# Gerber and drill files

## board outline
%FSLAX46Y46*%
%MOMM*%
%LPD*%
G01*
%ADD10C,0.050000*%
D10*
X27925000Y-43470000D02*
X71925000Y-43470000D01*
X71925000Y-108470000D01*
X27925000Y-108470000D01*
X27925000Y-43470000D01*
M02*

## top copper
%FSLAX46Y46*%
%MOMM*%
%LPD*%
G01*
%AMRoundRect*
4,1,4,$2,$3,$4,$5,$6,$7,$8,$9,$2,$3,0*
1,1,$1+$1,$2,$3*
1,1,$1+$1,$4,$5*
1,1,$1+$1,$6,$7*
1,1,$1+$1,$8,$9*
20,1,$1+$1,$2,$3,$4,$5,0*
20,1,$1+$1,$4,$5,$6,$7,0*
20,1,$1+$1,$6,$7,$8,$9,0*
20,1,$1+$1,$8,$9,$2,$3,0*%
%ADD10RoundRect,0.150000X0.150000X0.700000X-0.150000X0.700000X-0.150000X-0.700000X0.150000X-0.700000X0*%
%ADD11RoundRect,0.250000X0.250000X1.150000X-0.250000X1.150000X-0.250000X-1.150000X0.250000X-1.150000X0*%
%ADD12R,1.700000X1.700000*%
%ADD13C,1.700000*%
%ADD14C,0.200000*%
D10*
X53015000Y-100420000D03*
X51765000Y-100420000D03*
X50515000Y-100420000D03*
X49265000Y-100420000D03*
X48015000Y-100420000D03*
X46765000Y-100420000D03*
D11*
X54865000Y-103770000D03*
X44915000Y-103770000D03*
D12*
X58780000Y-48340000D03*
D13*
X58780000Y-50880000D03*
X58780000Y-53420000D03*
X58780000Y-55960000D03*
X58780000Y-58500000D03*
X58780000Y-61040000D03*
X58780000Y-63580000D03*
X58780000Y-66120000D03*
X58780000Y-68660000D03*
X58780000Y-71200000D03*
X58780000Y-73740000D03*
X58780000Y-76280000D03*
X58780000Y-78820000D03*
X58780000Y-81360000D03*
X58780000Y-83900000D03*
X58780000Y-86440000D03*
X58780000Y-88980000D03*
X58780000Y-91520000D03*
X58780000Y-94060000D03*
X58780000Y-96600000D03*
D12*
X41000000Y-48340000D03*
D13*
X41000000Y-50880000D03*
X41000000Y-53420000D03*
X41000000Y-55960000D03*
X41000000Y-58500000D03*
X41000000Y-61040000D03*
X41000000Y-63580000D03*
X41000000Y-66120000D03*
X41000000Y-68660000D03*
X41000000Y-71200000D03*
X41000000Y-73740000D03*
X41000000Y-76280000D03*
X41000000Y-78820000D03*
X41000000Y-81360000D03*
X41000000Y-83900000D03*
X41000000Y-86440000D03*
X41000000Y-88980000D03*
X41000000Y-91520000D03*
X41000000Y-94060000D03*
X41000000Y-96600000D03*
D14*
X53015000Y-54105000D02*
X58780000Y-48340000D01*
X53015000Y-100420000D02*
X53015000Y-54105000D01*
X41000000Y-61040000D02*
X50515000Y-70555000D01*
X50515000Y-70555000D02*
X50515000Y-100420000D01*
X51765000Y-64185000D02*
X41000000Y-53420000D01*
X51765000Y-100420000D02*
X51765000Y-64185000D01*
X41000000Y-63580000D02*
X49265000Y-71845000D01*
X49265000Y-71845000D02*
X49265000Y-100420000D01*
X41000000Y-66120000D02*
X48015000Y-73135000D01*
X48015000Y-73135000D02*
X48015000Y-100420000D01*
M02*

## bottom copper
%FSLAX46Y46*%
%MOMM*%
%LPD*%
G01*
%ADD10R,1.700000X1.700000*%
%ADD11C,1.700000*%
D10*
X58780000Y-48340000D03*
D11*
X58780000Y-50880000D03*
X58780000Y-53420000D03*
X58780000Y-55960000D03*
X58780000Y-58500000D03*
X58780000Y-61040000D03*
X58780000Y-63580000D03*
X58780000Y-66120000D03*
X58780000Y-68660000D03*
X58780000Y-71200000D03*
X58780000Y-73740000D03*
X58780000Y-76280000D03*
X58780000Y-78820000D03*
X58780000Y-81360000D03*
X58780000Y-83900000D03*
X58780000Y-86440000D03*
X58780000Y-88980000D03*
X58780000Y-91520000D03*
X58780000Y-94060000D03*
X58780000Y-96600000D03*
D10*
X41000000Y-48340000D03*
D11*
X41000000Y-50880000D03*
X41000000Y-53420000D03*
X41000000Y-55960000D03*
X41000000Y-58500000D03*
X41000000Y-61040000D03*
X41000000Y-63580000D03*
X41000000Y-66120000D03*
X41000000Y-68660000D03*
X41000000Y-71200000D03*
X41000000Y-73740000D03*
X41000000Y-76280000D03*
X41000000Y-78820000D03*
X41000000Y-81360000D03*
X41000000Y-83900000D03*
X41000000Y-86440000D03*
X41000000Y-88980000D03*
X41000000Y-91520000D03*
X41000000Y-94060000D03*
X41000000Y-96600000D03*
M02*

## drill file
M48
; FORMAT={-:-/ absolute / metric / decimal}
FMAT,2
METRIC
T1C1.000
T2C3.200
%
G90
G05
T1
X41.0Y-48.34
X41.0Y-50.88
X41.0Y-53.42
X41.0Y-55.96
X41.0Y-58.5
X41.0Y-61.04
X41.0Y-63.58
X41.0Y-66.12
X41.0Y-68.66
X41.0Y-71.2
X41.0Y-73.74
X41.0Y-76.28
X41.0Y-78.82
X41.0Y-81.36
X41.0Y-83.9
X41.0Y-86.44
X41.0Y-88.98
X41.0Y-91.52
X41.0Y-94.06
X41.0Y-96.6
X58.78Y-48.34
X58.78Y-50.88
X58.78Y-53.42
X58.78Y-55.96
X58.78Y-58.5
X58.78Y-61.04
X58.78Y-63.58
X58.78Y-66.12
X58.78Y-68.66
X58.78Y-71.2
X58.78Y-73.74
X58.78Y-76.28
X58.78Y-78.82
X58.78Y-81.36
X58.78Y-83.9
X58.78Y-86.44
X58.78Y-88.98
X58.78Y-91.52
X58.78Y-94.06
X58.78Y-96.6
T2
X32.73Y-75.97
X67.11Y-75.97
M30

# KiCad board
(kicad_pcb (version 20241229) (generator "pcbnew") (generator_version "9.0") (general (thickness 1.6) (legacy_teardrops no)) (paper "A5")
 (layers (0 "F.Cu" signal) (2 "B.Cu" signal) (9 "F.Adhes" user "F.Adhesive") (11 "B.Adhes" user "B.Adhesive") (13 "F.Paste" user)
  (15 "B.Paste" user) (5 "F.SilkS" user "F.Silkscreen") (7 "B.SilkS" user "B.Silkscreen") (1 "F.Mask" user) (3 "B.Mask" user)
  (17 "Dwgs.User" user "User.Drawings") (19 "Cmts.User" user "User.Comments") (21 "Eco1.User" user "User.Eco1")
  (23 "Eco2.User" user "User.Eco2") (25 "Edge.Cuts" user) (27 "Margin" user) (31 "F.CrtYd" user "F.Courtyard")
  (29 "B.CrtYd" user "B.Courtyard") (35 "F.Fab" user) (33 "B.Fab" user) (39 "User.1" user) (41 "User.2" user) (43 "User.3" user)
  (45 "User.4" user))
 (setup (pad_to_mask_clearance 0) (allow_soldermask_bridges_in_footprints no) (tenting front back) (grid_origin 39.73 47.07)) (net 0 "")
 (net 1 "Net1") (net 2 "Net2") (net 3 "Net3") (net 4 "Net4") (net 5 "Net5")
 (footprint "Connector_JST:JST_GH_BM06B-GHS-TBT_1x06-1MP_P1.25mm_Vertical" (layer "F.Cu") (at 49.89 102.37 180)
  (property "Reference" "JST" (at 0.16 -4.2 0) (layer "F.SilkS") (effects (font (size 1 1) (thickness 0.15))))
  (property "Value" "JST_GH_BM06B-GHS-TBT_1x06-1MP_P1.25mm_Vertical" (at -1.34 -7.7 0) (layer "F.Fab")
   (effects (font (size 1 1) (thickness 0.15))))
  (pad "1" smd roundrect (at -3.125 1.95 180) (size 0.6 1.7) (layers "F.Cu" "F.Mask" "F.Paste") (roundrect_rratio 0.25) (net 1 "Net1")
   (solder_mask_margin 0))
  (pad "2" smd roundrect (at -1.875 1.95 180) (size 0.6 1.7) (layers "F.Cu" "F.Mask" "F.Paste") (roundrect_rratio 0.25) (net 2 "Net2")
   (solder_mask_margin 0))
  (pad "3" smd roundrect (at -0.625 1.95 180) (size 0.6 1.7) (layers "F.Cu" "F.Mask" "F.Paste") (roundrect_rratio 0.25) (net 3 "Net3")
   (solder_mask_margin 0))
  (pad "4" smd roundrect (at 0.625 1.95 180) (size 0.6 1.7) (layers "F.Cu" "F.Mask" "F.Paste") (roundrect_rratio 0.25) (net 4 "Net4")
   (solder_mask_margin 0))
  (pad "5" smd roundrect (at 1.875 1.95 180) (size 0.6 1.7) (layers "F.Cu" "F.Mask" "F.Paste") (roundrect_rratio 0.25) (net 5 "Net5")
   (solder_mask_margin 0))
  (pad "6" smd roundrect (at 3.125 1.95 180) (size 0.6 1.7) (layers "F.Cu" "F.Mask" "F.Paste") (roundrect_rratio 0.25))
  (pad "MP" smd roundrect (at -4.975 -1.4 180) (size 1 2.8) (layers "F.Cu" "F.Mask" "F.Paste") (roundrect_rratio 0.25))
  (pad "MP" smd roundrect (at 4.975 -1.4 180) (size 1 2.8) (layers "F.Cu" "F.Mask" "F.Paste") (roundrect_rratio 0.25)))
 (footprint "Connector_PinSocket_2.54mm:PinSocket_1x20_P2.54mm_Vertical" (layer "F.Cu") (at 58.78 48.34)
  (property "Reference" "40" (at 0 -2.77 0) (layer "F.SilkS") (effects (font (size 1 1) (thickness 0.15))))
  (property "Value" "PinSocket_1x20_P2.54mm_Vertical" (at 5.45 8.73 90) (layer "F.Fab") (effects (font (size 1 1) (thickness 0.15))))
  (pad "1" thru_hole rect (at 0 0) (size 1.7 1.7) (drill 1) (layers "*.Cu" "*.Mask") (remove_unused_layers no) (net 1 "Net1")
   (solder_mask_margin 0))
  (pad "2" thru_hole circle (at 0 2.54) (size 1.7 1.7) (drill 1) (layers "*.Cu" "*.Mask") (remove_unused_layers no))
  (pad "3" thru_hole circle (at 0 5.08) (size 1.7 1.7) (drill 1) (layers "*.Cu" "*.Mask") (remove_unused_layers no))
  (pad "4" thru_hole circle (at 0 7.62) (size 1.7 1.7) (drill 1) (layers "*.Cu" "*.Mask") (remove_unused_layers no))
  (pad "5" thru_hole circle (at 0 10.16) (size 1.7 1.7) (drill 1) (layers "*.Cu" "*.Mask") (remove_unused_layers no))
  (pad "6" thru_hole circle (at 0 12.7) (size 1.7 1.7) (drill 1) (layers "*.Cu" "*.Mask") (remove_unused_layers no))
  (pad "7" thru_hole circle (at 0 15.24) (size 1.7 1.7) (drill 1) (layers "*.Cu" "*.Mask") (remove_unused_layers no))
  (pad "8" thru_hole circle (at 0 17.78) (size 1.7 1.7) (drill 1) (layers "*.Cu" "*.Mask") (remove_unused_layers no))
  (pad "9" thru_hole circle (at 0 20.32) (size 1.7 1.7) (drill 1) (layers "*.Cu" "*.Mask") (remove_unused_layers no))
  (pad "10" thru_hole circle (at 0 22.86) (size 1.7 1.7) (drill 1) (layers "*.Cu" "*.Mask") (remove_unused_layers no))
  (pad "11" thru_hole circle (at 0 25.4) (size 1.7 1.7) (drill 1) (layers "*.Cu" "*.Mask") (remove_unused_layers no))
  (pad "12" thru_hole circle (at 0 27.94) (size 1.7 1.7) (drill 1) (layers "*.Cu" "*.Mask") (remove_unused_layers no))
  (pad "13" thru_hole circle (at 0 30.48) (size 1.7 1.7) (drill 1) (layers "*.Cu" "*.Mask") (remove_unused_layers no))
  (pad "14" thru_hole circle (at 0 33.02) (size 1.7 1.7) (drill 1) (layers "*.Cu" "*.Mask") (remove_unused_layers no))
  (pad "15" thru_hole circle (at 0 35.56) (size 1.7 1.7) (drill 1) (layers "*.Cu" "*.Mask") (remove_unused_layers no))
  (pad "16" thru_hole circle (at 0 38.1) (size 1.7 1.7) (drill 1) (layers "*.Cu" "*.Mask") (remove_unused_layers no))
  (pad "17" thru_hole circle (at 0 40.64) (size 1.7 1.7) (drill 1) (layers "*.Cu" "*.Mask") (remove_unused_layers no))
  (pad "18" thru_hole circle (at 0 43.18) (size 1.7 1.7) (drill 1) (layers "*.Cu" "*.Mask") (remove_unused_layers no))
  (pad "19" thru_hole circle (at 0 45.72) (size 1.7 1.7) (drill 1) (layers "*.Cu" "*.Mask") (remove_unused_layers no))
  (pad "20" thru_hole circle (at 0 48.26) (size 1.7 1.7) (drill 1) (layers "*.Cu" "*.Mask") (remove_unused_layers no)))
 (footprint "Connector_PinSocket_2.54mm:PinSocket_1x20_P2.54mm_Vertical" (layer "F.Cu") (at 41 48.34)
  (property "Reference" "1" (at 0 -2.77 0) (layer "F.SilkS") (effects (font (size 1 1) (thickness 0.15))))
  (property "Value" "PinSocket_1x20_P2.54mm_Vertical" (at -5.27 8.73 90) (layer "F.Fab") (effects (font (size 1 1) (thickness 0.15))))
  (pad "1" thru_hole rect (at 0 0) (size 1.7 1.7) (drill 1) (layers "*.Cu" "*.Mask") (remove_unused_layers no))
  (pad "2" thru_hole circle (at 0 2.54) (size 1.7 1.7) (drill 1) (layers "*.Cu" "*.Mask") (remove_unused_layers no))
  (pad "3" thru_hole circle (at 0 5.08) (size 1.7 1.7) (drill 1) (layers "*.Cu" "*.Mask") (remove_unused_layers no) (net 2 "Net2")
   (solder_mask_margin 0))
  (pad "4" thru_hole circle (at 0 7.62) (size 1.7 1.7) (drill 1) (layers "*.Cu" "*.Mask") (remove_unused_layers no))
  (pad "5" thru_hole circle (at 0 10.16) (size 1.7 1.7) (drill 1) (layers "*.Cu" "*.Mask") (remove_unused_layers no))
  (pad "6" thru_hole circle (at 0 12.7) (size 1.7 1.7) (drill 1) (layers "*.Cu" "*.Mask") (remove_unused_layers no) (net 3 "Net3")
   (solder_mask_margin 0))
  (pad "7" thru_hole circle (at 0 15.24) (size 1.7 1.7) (drill 1) (layers "*.Cu" "*.Mask") (remove_unused_layers no) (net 4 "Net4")
   (clearance 0))
  (pad "8" thru_hole circle (at 0 17.78) (size 1.7 1.7) (drill 1) (layers "*.Cu" "*.Mask") (remove_unused_layers no) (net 5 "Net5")
   (solder_mask_margin 0))
  (pad "9" thru_hole circle (at 0 20.32) (size 1.7 1.7) (drill 1) (layers "*.Cu" "*.Mask") (remove_unused_layers no))
  (pad "10" thru_hole circle (at 0 22.86) (size 1.7 1.7) (drill 1) (layers "*.Cu" "*.Mask") (remove_unused_layers no))
  (pad "11" thru_hole circle (at 0 25.4) (size 1.7 1.7) (drill 1) (layers "*.Cu" "*.Mask") (remove_unused_layers no))
  (pad "12" thru_hole circle (at 0 27.94) (size 1.7 1.7) (drill 1) (layers "*.Cu" "*.Mask") (remove_unused_layers no))
  (pad "13" thru_hole circle (at 0 30.48) (size 1.7 1.7) (drill 1) (layers "*.Cu" "*.Mask") (remove_unused_layers no))
  (pad "14" thru_hole circle (at 0 33.02) (size 1.7 1.7) (drill 1) (layers "*.Cu" "*.Mask") (remove_unused_layers no))
  (pad "15" thru_hole circle (at 0 35.56) (size 1.7 1.7) (drill 1) (layers "*.Cu" "*.Mask") (remove_unused_layers no))
  (pad "16" thru_hole circle (at 0 38.1) (size 1.7 1.7) (drill 1) (layers "*.Cu" "*.Mask") (remove_unused_layers no))
  (pad "17" thru_hole circle (at 0 40.64) (size 1.7 1.7) (drill 1) (layers "*.Cu" "*.Mask") (remove_unused_layers no))
  (pad "18" thru_hole circle (at 0 43.18) (size 1.7 1.7) (drill 1) (layers "*.Cu" "*.Mask") (remove_unused_layers no))
  (pad "19" thru_hole circle (at 0 45.72) (size 1.7 1.7) (drill 1) (layers "*.Cu" "*.Mask") (remove_unused_layers no))
  (pad "20" thru_hole circle (at 0 48.26) (size 1.7 1.7) (drill 1) (layers "*.Cu" "*.Mask") (remove_unused_layers no)))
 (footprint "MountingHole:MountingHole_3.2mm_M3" (layer "F.Cu") (at 32.73 75.97)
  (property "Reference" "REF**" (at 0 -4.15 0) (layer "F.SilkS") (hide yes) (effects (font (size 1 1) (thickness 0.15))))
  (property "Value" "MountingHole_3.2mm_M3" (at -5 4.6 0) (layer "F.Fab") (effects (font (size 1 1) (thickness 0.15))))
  (pad "" np_thru_hole circle (at 0 0) (size 3.2 3.2) (drill 3.2) (layers "*.Cu" "*.Mask")))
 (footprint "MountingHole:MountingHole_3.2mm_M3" (layer "F.Cu") (at 67.11 75.97)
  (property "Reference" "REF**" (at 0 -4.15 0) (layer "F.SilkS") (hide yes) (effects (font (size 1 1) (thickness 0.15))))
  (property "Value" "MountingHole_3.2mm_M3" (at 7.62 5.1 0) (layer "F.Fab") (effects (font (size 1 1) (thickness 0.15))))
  (pad "" np_thru_hole circle (at 0 0) (size 3.2 3.2) (drill 3.2) (layers "*.Cu" "*.Mask")))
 (gr_rect (start 27.925 43.47) (end 71.925 108.47) (stroke (width 0.05) (type solid)) (fill no) (layer "Edge.Cuts"))
 (segment (start 53.015 54.105) (end 58.78 48.34) (width 0.2) (layer "F.Cu") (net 1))
 (segment (start 53.015 100.42) (end 53.015 54.105) (width 0.2) (layer "F.Cu") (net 1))
 (segment (start 41 61.04) (end 50.515 70.555) (width 0.2) (layer "F.Cu") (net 3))
 (segment (start 50.515 70.555) (end 50.515 100.42) (width 0.2) (layer "F.Cu") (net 3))
 (segment (start 51.765 64.185) (end 41 53.42) (width 0.2) (layer "F.Cu") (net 2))
 (segment (start 51.765 100.42) (end 51.765 64.185) (width 0.2) (layer "F.Cu") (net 2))
 (segment (start 41 63.58) (end 49.265 71.845) (width 0.2) (layer "F.Cu") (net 4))
 (segment (start 49.265 71.845) (end 49.265 100.42) (width 0.2) (layer "F.Cu") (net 4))
 (segment (start 41 66.12) (end 48.015 73.135) (width 0.2) (layer "F.Cu") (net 5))
 (segment (start 48.015 73.135) (end 48.015 100.42) (width 0.2) (layer "F.Cu") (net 5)))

